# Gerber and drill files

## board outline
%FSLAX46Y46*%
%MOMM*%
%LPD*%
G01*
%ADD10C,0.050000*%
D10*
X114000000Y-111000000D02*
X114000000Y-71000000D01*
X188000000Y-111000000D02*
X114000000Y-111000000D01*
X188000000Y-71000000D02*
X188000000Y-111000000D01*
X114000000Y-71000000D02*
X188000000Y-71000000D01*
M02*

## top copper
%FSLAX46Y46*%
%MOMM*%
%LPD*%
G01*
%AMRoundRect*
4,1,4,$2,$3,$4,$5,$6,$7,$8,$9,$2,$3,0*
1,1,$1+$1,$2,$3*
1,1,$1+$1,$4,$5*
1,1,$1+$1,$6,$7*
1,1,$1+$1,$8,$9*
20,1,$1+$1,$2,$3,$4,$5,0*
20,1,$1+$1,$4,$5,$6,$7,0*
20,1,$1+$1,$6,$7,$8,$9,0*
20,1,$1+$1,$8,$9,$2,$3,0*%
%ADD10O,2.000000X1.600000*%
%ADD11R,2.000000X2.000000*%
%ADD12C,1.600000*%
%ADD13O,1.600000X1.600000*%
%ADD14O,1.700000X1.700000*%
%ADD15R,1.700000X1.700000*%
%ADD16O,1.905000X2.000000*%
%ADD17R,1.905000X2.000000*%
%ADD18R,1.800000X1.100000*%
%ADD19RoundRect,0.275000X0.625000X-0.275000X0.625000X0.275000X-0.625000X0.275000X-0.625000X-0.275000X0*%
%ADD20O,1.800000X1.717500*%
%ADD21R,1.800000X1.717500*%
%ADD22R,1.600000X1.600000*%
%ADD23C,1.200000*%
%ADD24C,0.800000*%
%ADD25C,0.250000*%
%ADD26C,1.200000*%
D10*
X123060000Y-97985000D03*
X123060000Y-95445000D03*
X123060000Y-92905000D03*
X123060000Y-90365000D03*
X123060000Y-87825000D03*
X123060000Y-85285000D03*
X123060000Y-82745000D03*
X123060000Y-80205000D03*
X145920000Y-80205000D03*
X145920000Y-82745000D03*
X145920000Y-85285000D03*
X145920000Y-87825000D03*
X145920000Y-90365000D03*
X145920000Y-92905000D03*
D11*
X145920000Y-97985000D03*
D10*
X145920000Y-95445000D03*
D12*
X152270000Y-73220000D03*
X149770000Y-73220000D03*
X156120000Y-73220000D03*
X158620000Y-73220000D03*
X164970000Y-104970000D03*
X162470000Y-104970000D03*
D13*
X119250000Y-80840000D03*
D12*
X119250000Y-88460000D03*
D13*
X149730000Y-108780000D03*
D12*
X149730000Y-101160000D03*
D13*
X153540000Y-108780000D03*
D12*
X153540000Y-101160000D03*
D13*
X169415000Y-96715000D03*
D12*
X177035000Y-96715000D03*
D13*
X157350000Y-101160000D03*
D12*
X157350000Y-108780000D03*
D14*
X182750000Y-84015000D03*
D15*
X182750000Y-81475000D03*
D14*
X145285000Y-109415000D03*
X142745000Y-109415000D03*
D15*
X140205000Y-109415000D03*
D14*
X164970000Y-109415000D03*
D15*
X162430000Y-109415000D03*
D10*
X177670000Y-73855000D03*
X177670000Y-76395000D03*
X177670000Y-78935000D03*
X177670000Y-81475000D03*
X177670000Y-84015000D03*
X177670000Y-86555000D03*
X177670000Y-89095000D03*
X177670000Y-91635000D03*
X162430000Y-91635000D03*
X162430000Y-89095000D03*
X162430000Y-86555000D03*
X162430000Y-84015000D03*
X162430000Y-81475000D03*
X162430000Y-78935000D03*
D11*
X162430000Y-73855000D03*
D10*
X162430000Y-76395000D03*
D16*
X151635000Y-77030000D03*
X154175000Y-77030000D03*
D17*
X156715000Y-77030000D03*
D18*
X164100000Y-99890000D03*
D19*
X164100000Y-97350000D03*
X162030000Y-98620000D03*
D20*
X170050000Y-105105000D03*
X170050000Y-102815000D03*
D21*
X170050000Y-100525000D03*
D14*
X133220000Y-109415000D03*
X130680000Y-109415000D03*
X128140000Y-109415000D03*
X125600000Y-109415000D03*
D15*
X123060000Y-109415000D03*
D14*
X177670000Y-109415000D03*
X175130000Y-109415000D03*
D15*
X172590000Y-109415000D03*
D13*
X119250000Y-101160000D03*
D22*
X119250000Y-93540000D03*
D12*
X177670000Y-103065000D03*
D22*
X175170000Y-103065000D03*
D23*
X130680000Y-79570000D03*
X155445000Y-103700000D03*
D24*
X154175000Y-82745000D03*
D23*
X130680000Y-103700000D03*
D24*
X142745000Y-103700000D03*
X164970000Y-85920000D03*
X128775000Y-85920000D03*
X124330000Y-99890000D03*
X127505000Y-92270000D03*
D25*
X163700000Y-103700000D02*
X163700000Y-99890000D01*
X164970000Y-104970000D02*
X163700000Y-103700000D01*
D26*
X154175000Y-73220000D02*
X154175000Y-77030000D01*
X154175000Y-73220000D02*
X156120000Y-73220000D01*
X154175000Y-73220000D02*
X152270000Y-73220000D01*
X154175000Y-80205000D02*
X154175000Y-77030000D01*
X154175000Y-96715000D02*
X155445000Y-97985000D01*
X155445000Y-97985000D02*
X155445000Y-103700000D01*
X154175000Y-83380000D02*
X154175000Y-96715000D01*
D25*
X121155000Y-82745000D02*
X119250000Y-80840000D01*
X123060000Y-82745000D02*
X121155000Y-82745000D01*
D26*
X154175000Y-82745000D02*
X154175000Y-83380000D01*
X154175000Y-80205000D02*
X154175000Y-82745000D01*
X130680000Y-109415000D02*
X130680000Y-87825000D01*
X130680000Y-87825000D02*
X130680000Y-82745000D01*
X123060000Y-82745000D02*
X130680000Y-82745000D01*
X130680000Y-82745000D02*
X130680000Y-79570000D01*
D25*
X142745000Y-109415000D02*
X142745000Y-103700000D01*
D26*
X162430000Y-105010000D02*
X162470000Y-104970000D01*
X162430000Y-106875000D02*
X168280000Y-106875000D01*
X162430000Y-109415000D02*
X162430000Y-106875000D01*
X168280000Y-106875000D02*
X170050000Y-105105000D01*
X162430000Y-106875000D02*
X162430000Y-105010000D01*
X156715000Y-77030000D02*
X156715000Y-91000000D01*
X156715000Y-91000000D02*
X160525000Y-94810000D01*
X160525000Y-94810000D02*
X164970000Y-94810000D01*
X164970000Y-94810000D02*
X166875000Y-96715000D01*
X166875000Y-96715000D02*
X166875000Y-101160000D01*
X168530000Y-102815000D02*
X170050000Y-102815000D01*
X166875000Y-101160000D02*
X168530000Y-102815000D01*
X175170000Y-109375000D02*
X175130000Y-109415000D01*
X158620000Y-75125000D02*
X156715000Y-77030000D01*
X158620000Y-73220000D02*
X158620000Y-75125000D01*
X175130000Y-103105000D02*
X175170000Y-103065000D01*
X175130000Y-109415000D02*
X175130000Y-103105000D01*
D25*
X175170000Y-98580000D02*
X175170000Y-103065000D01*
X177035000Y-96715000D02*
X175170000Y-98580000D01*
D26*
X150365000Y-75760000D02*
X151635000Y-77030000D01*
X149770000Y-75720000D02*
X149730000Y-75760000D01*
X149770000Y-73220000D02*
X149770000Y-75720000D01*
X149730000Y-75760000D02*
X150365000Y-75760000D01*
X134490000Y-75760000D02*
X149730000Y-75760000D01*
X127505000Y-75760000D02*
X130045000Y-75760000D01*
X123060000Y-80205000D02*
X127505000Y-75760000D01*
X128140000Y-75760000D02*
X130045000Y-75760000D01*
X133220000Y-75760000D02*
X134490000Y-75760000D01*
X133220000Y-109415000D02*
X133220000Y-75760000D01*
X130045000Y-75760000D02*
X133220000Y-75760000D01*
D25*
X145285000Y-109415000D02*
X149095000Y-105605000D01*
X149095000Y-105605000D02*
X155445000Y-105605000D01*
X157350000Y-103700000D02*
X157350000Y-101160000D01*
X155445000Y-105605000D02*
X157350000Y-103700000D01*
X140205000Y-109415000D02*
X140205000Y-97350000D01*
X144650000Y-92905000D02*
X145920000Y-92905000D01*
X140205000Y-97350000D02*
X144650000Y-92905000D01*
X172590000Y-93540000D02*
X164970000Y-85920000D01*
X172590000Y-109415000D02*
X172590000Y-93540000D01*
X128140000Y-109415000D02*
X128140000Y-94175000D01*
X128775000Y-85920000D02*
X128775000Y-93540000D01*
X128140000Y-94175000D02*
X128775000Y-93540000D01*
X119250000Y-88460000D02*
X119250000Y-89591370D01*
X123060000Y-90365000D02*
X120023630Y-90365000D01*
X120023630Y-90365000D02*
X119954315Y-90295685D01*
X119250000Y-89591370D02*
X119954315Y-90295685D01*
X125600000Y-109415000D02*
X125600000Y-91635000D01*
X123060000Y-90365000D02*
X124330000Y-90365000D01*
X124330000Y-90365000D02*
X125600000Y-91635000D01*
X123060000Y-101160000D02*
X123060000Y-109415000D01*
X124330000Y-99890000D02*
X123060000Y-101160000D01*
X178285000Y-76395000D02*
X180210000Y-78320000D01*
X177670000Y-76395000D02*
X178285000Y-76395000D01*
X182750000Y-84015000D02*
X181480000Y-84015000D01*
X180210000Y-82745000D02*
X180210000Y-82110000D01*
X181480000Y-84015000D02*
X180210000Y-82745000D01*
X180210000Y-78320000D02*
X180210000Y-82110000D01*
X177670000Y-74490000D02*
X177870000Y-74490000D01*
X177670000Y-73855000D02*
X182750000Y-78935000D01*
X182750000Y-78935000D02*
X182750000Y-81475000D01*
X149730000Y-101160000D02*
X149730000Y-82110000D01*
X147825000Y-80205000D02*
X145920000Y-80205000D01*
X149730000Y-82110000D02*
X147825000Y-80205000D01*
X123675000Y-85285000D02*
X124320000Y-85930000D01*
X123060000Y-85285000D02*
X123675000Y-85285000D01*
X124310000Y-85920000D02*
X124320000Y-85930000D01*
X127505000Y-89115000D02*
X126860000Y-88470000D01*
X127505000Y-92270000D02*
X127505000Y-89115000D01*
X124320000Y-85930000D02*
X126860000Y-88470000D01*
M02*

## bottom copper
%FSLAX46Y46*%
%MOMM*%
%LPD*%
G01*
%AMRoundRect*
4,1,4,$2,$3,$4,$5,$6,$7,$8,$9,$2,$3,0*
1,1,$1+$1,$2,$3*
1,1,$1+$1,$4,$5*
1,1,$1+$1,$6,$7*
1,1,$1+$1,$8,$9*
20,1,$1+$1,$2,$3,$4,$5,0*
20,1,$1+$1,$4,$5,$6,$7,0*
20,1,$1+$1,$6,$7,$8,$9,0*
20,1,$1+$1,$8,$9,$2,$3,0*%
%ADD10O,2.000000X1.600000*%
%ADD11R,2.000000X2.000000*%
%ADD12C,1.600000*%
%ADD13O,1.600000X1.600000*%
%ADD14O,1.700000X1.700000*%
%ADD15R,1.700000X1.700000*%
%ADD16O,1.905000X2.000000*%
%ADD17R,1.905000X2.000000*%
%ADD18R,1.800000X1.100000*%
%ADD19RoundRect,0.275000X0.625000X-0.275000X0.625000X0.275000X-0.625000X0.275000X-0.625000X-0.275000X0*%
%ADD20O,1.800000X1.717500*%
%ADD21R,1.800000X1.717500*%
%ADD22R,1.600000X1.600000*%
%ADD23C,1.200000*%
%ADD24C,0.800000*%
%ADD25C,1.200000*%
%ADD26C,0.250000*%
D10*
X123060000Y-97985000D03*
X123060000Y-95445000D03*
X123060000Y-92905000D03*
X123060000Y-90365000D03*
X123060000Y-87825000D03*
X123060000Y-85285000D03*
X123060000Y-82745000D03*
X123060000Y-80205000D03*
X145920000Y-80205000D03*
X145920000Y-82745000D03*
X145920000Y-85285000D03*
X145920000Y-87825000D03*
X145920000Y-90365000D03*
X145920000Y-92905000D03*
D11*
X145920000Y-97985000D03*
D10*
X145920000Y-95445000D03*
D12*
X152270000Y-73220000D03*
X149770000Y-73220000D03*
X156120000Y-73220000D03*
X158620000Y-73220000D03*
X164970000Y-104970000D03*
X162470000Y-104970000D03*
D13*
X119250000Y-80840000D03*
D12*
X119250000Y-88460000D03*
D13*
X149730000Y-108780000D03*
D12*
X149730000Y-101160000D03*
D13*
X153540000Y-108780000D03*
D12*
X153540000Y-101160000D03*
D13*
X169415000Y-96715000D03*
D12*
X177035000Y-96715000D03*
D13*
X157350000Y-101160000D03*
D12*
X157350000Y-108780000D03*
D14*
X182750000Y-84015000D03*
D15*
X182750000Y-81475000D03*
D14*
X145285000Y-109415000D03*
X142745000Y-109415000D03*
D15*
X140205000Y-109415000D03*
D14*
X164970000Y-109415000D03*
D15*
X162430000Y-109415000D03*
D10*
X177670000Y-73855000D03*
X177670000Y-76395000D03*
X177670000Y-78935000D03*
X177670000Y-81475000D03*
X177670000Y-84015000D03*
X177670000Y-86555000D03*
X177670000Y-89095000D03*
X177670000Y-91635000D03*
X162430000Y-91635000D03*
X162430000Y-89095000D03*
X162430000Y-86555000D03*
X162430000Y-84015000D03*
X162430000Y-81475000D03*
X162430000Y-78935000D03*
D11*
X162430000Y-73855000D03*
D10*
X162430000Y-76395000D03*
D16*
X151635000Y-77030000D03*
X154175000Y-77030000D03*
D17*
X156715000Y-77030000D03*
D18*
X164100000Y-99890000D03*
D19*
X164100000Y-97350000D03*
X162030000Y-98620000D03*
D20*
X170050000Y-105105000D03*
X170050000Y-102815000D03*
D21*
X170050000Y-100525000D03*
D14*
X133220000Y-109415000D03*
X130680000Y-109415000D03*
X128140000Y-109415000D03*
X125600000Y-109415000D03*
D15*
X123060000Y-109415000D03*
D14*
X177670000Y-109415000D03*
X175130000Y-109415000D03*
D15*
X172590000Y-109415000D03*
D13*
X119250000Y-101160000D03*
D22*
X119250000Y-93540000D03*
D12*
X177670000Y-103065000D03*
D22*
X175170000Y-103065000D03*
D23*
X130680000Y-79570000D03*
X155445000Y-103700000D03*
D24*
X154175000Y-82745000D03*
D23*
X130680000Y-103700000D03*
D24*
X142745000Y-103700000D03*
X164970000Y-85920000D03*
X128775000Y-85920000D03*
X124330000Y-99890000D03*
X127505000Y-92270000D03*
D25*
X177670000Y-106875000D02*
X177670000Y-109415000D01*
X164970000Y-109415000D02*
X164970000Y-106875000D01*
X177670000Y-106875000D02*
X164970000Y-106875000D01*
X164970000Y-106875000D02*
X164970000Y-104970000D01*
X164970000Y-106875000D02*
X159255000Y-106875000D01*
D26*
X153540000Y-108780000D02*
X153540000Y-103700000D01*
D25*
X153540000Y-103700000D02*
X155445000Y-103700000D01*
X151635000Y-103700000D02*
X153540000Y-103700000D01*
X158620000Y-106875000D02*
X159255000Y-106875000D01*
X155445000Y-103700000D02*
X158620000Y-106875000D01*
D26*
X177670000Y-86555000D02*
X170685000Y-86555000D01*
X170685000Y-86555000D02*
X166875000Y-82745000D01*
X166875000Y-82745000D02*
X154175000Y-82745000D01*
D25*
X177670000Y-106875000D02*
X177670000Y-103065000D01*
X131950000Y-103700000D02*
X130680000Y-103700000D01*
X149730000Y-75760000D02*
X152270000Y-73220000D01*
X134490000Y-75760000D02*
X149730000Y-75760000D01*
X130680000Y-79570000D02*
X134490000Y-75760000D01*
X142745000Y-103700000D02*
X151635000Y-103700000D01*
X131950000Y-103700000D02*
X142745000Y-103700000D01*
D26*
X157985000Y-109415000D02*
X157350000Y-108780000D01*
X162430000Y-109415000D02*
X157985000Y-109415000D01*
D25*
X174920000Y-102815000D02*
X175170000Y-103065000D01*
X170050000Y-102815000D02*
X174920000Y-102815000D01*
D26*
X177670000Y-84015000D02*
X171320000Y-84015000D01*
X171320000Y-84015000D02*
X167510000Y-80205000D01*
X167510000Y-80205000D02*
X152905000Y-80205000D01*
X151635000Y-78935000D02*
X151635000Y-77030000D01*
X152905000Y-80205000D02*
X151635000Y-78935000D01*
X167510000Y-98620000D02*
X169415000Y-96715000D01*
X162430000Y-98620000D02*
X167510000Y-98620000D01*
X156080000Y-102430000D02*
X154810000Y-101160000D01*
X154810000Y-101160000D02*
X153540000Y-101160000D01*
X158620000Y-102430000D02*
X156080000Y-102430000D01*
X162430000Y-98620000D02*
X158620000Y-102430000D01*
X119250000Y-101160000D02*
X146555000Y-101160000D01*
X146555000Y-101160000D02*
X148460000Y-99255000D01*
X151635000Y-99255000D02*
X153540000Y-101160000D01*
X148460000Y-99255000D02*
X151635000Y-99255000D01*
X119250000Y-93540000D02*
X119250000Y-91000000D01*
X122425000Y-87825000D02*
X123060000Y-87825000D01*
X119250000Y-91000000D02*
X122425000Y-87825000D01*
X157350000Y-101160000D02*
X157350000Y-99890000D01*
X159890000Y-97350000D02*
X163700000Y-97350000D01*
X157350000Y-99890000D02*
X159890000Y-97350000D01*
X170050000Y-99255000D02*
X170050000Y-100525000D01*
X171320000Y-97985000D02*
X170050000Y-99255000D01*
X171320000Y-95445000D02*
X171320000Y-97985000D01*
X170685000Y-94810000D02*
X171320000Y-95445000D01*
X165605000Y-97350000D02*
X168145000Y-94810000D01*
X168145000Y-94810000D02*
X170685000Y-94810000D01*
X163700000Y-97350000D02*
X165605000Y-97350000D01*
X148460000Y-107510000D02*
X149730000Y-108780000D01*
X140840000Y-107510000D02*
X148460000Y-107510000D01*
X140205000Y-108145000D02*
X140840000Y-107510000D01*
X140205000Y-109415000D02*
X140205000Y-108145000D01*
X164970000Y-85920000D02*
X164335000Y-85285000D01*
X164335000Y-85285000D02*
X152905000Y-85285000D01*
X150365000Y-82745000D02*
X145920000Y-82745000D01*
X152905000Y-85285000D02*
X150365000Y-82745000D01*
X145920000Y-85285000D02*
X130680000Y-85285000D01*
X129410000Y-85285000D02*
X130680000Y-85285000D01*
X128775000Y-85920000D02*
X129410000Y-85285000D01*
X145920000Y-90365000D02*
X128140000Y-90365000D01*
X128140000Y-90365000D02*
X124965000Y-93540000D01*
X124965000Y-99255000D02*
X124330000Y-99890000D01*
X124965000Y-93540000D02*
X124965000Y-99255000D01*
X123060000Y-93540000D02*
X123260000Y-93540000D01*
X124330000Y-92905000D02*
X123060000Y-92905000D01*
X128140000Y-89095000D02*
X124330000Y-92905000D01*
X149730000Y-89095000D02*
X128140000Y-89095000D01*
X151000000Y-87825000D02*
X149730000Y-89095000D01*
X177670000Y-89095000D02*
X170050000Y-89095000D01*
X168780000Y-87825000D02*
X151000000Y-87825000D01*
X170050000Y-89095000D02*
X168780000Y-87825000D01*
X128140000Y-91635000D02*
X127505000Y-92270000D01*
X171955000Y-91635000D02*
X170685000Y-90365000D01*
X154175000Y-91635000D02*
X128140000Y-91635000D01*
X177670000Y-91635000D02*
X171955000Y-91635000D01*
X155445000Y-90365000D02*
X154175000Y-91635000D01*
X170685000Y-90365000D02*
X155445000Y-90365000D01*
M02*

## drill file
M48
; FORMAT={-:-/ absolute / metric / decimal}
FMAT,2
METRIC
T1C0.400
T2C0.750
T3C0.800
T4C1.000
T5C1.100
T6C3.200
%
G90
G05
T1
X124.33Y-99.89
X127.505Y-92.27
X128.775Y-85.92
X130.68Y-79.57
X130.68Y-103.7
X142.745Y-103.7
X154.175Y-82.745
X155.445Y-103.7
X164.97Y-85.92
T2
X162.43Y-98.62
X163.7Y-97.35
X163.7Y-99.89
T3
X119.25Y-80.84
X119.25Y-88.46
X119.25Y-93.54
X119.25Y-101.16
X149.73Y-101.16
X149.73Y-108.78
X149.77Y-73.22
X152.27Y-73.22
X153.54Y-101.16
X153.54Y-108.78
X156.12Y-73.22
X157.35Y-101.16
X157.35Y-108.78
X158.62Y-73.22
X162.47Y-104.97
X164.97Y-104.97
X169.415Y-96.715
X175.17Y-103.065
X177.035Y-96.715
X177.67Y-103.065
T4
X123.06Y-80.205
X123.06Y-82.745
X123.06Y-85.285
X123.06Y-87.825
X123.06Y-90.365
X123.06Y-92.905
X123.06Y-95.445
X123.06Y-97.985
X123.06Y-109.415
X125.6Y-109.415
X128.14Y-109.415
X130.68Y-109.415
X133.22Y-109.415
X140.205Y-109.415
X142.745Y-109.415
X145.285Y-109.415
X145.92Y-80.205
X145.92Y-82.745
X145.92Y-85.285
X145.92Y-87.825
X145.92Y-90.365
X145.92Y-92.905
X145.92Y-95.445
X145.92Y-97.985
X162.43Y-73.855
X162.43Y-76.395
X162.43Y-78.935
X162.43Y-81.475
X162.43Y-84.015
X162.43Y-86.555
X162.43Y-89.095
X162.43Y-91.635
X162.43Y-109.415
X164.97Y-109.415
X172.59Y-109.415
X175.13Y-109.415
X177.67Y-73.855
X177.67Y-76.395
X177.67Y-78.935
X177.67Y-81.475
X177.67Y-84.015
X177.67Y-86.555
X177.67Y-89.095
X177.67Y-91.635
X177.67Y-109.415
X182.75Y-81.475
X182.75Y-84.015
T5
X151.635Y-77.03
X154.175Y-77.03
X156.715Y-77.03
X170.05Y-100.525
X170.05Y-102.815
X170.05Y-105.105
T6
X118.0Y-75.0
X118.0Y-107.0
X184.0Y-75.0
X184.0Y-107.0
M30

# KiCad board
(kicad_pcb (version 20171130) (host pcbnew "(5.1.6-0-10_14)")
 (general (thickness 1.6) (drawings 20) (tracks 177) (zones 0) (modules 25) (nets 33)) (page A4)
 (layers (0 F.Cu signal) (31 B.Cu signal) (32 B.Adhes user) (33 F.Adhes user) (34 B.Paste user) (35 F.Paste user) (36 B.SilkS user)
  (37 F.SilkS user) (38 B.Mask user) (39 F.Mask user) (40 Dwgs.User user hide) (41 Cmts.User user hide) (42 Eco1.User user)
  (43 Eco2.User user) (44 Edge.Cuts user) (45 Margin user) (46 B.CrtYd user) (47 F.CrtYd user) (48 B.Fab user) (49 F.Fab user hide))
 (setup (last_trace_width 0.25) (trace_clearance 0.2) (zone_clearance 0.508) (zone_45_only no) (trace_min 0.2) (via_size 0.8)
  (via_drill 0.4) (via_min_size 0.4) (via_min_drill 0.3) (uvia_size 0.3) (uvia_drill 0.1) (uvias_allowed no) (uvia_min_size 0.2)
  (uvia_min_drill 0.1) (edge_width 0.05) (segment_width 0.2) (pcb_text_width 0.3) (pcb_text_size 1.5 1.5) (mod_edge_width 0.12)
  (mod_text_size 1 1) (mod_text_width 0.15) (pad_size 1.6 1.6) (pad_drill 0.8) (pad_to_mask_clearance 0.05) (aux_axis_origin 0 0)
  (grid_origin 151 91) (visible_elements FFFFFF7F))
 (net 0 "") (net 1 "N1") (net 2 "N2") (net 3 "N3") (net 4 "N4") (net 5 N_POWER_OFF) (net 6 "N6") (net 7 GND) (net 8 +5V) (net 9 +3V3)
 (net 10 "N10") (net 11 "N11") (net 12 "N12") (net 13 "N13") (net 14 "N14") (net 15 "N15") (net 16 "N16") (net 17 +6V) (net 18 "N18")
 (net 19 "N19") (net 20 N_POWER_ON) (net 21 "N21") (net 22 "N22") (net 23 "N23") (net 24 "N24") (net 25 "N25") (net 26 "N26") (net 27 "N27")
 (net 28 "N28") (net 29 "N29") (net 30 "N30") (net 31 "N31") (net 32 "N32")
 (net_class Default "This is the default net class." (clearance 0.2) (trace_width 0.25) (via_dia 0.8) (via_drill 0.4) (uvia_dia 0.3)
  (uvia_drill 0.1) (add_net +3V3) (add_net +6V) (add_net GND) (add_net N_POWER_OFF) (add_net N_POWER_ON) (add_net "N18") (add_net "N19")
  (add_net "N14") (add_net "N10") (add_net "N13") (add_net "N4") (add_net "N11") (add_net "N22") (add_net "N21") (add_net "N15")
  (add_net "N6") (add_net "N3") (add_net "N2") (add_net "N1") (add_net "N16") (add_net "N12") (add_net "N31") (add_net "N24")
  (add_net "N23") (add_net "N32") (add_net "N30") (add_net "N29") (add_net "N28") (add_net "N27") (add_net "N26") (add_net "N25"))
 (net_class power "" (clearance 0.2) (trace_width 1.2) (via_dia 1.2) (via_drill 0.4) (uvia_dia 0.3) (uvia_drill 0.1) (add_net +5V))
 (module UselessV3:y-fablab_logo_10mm (layer F.Cu) (at 154.175 88.46)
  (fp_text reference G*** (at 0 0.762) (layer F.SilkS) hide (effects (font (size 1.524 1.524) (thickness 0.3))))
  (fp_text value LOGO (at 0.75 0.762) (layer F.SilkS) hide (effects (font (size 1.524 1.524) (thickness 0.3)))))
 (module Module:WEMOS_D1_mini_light (layer F.Cu) (at 145.92 97.985 180)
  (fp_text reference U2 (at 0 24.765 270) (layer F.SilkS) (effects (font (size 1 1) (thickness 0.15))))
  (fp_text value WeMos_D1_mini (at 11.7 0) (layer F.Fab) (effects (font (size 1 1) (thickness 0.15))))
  (pad 16 thru_hole oval (at 22.86 0 180) (size 2 1.6) (drill 1) (layers *.Cu *.Mask) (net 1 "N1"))
  (pad 15 thru_hole oval (at 22.86 2.54 180) (size 2 1.6) (drill 1) (layers *.Cu *.Mask) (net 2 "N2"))
  (pad 14 thru_hole oval (at 22.86 5.08 180) (size 2 1.6) (drill 1) (layers *.Cu *.Mask) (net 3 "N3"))
  (pad 13 thru_hole oval (at 22.86 7.62 180) (size 2 1.6) (drill 1) (layers *.Cu *.Mask) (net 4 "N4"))
  (pad 12 thru_hole oval (at 22.86 10.16 180) (size 2 1.6) (drill 1) (layers *.Cu *.Mask) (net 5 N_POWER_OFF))
  (pad 11 thru_hole oval (at 22.86 12.7 180) (size 2 1.6) (drill 1) (layers *.Cu *.Mask) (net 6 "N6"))
  (pad 10 thru_hole oval (at 22.86 15.24 180) (size 2 1.6) (drill 1) (layers *.Cu *.Mask) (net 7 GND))
  (pad 9 thru_hole oval (at 22.86 17.78 180) (size 2 1.6) (drill 1) (layers *.Cu *.Mask) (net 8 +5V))
  (pad 8 thru_hole oval (at 0 17.78 180) (size 2 1.6) (drill 1) (layers *.Cu *.Mask) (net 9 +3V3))
  (pad 7 thru_hole oval (at 0 15.24 180) (size 2 1.6) (drill 1) (layers *.Cu *.Mask) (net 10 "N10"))
  (pad 6 thru_hole oval (at 0 12.7 180) (size 2 1.6) (drill 1) (layers *.Cu *.Mask) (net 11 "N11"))
  (pad 5 thru_hole oval (at 0 10.16 180) (size 2 1.6) (drill 1) (layers *.Cu *.Mask) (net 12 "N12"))
  (pad 4 thru_hole oval (at 0 7.62 180) (size 2 1.6) (drill 1) (layers *.Cu *.Mask) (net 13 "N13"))
  (pad 3 thru_hole oval (at 0 5.08 180) (size 2 1.6) (drill 1) (layers *.Cu *.Mask) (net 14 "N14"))
  (pad 1 thru_hole rect (at 0 0 180) (size 2 2) (drill 1) (layers *.Cu *.Mask) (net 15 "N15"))
  (pad 2 thru_hole oval (at 0 2.54 180) (size 2 1.6) (drill 1) (layers *.Cu *.Mask) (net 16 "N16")))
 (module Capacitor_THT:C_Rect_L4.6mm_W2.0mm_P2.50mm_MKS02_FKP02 (layer F.Cu) (at 149.77 73.22)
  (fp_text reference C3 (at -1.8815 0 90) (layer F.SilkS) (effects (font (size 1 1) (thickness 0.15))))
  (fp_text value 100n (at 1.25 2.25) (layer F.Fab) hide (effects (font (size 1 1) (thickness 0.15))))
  (pad 2 thru_hole circle (at 2.5 0) (size 1.6 1.6) (drill 0.8) (layers *.Cu *.Mask) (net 7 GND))
  (pad 1 thru_hole circle (at 0 0) (size 1.6 1.6) (drill 0.8) (layers *.Cu *.Mask) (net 8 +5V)))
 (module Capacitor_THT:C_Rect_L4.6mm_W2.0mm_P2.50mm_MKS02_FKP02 (layer F.Cu) (at 158.62 73.22 180)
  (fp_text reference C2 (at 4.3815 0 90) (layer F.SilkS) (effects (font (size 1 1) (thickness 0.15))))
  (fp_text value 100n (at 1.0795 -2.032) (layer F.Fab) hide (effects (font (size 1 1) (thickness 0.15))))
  (pad 2 thru_hole circle (at 2.5 0 180) (size 1.6 1.6) (drill 0.8) (layers *.Cu *.Mask) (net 7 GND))
  (pad 1 thru_hole circle (at 0 0 180) (size 1.6 1.6) (drill 0.8) (layers *.Cu *.Mask) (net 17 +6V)))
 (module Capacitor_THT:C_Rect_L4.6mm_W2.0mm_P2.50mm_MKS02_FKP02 (layer F.Cu) (at 162.47 104.97)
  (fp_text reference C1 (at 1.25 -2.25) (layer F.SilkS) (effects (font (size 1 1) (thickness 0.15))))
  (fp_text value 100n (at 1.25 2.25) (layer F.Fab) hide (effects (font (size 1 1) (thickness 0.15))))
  (pad 2 thru_hole circle (at 2.5 0) (size 1.6 1.6) (drill 0.8) (layers *.Cu *.Mask) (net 7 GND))
  (pad 1 thru_hole circle (at 0 0) (size 1.6 1.6) (drill 0.8) (layers *.Cu *.Mask) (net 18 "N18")))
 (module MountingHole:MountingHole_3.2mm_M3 (layer F.Cu) (at 184 75)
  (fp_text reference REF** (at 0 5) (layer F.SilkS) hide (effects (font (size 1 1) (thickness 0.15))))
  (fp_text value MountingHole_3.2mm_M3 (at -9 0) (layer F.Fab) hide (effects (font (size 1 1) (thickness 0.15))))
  (pad 1 np_thru_hole circle (at 0 0) (size 3.2 3.2) (drill 3.2) (layers *.Cu *.Mask)))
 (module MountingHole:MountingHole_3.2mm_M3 (layer F.Cu) (at 184 107)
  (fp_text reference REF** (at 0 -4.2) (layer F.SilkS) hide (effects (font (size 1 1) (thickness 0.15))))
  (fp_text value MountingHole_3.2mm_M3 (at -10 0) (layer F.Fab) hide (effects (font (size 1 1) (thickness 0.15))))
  (pad 1 np_thru_hole circle (at 0 0) (size 3.2 3.2) (drill 3.2) (layers *.Cu *.Mask)))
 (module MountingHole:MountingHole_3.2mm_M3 (layer F.Cu) (at 118 107)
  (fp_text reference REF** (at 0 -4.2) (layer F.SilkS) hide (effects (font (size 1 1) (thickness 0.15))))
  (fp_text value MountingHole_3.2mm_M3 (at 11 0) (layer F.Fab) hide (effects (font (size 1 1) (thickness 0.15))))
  (pad 1 np_thru_hole circle (at 0 0) (size 3.2 3.2) (drill 3.2) (layers *.Cu *.Mask)))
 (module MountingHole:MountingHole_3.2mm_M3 (layer F.Cu) (at 118 75)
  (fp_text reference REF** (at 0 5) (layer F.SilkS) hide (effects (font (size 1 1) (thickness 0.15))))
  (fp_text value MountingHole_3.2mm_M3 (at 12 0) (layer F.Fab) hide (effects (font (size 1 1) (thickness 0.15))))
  (pad 1 np_thru_hole circle (at 0 0) (size 3.2 3.2) (drill 3.2) (layers *.Cu *.Mask)))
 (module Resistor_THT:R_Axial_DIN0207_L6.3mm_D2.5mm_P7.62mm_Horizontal (layer F.Cu) (at 119.25 88.46 90)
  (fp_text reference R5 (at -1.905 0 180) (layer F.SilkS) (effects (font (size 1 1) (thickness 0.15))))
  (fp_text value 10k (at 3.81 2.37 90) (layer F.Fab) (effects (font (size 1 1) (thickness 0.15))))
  (pad 2 thru_hole oval (at 7.62 0 90) (size 1.6 1.6) (drill 0.8) (layers *.Cu *.Mask) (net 7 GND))
  (pad 1 thru_hole circle (at 0 0 90) (size 1.6 1.6) (drill 0.8) (layers *.Cu *.Mask) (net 4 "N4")))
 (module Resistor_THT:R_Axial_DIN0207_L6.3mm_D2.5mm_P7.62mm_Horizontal (layer F.Cu) (at 149.73 101.16 270)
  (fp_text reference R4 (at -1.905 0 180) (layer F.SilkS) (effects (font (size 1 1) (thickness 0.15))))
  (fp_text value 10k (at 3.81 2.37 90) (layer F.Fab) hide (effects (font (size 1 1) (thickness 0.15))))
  (pad 2 thru_hole oval (at 7.62 0 270) (size 1.6 1.6) (drill 0.8) (layers *.Cu *.Mask) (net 14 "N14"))
  (pad 1 thru_hole circle (at 0 0 270) (size 1.6 1.6) (drill 0.8) (layers *.Cu *.Mask) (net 9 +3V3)))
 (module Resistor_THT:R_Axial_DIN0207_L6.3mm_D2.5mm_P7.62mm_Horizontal (layer F.Cu) (at 153.54 101.16 270)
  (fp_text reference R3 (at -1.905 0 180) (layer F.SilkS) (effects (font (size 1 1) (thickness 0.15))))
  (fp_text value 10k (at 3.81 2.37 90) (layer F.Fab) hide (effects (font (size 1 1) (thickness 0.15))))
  (pad 2 thru_hole oval (at 7.62 0 270) (size 1.6 1.6) (drill 0.8) (layers *.Cu *.Mask) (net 7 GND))
  (pad 1 thru_hole circle (at 0 0 270) (size 1.6 1.6) (drill 0.8) (layers *.Cu *.Mask) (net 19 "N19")))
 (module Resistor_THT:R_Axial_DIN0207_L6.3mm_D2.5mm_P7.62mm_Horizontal (layer F.Cu) (at 177.035 96.715 180)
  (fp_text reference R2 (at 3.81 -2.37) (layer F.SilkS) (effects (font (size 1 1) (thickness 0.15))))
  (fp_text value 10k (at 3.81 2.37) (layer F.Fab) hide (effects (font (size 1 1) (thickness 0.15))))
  (pad 2 thru_hole oval (at 7.62 0 180) (size 1.6 1.6) (drill 0.8) (layers *.Cu *.Mask) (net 19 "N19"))
  (pad 1 thru_hole circle (at 0 0 180) (size 1.6 1.6) (drill 0.8) (layers *.Cu *.Mask) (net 17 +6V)))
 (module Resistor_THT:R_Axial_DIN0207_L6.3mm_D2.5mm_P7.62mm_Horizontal (layer F.Cu) (at 157.35 108.78 90)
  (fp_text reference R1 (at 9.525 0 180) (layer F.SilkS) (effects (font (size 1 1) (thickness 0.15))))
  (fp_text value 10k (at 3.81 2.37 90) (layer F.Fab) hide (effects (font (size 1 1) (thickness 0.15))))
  (pad 2 thru_hole oval (at 7.62 0 90) (size 1.6 1.6) (drill 0.8) (layers *.Cu *.Mask) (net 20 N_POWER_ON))
  (pad 1 thru_hole circle (at 0 0 90) (size 1.6 1.6) (drill 0.8) (layers *.Cu *.Mask) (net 18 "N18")))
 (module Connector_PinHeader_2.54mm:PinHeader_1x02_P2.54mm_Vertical (layer F.Cu) (at 182.75 81.475)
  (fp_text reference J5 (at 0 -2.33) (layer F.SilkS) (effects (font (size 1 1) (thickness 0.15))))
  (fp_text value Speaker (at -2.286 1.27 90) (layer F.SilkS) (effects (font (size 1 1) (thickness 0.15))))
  (pad 2 thru_hole oval (at 0 2.54) (size 1.7 1.7) (drill 1) (layers *.Cu *.Mask) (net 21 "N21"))
  (pad 1 thru_hole rect (at 0 0) (size 1.7 1.7) (drill 1) (layers *.Cu *.Mask) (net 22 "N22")))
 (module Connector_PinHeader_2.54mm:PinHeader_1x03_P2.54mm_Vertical (layer F.Cu) (at 140.205 109.415 90)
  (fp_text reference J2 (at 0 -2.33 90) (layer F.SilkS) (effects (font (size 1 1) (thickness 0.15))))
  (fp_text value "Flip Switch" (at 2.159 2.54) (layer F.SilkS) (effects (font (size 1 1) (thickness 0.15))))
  (pad 3 thru_hole oval (at 0 5.08 90) (size 1.7 1.7) (drill 1) (layers *.Cu *.Mask) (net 20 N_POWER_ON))
  (pad 2 thru_hole oval (at 0 2.54 90) (size 1.7 1.7) (drill 1) (layers *.Cu *.Mask) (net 7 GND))
  (pad 1 thru_hole rect (at 0 0 90) (size 1.7 1.7) (drill 1) (layers *.Cu *.Mask) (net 14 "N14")))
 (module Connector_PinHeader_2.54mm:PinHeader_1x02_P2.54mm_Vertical (layer F.Cu) (at 162.43 109.415 90)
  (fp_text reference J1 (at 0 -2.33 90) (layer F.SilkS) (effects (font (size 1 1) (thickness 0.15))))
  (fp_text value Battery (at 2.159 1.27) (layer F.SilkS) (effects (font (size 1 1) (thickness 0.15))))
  (pad 2 thru_hole oval (at 0 2.54 90) (size 1.7 1.7) (drill 1) (layers *.Cu *.Mask) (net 7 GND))
  (pad 1 thru_hole rect (at 0 0 90) (size 1.7 1.7) (drill 1) (layers *.Cu *.Mask) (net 18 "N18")))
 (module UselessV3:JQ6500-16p (layer F.Cu) (at 162.43 73.855)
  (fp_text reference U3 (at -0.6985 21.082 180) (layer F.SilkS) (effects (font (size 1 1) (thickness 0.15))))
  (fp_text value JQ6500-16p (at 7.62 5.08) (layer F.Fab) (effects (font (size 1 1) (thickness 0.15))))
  (pad 16 thru_hole oval (at 15.24 0) (size 2 1.6) (drill 1) (layers *.Cu *.Mask) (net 22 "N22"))
  (pad 15 thru_hole oval (at 15.24 2.54) (size 2 1.6) (drill 1) (layers *.Cu *.Mask) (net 21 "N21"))
  (pad 14 thru_hole oval (at 15.24 5.08) (size 2 1.6) (drill 1) (layers *.Cu *.Mask) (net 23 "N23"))
  (pad 13 thru_hole oval (at 15.24 7.62) (size 2 1.6) (drill 1) (layers *.Cu *.Mask) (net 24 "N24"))
  (pad 12 thru_hole oval (at 15.24 10.16) (size 2 1.6) (drill 1) (layers *.Cu *.Mask) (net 8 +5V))
  (pad 11 thru_hole oval (at 15.24 12.7) (size 2 1.6) (drill 1) (layers *.Cu *.Mask) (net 7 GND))
  (pad 10 thru_hole oval (at 15.24 15.24) (size 2 1.6) (drill 1) (layers *.Cu *.Mask) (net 3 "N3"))
  (pad 9 thru_hole oval (at 15.24 17.78) (size 2 1.6) (drill 1) (layers *.Cu *.Mask) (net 6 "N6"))
  (pad 8 thru_hole oval (at 0 17.78) (size 2 1.6) (drill 1) (layers *.Cu *.Mask) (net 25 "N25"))
  (pad 7 thru_hole oval (at 0 15.24) (size 2 1.6) (drill 1) (layers *.Cu *.Mask) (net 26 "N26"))
  (pad 6 thru_hole oval (at 0 12.7) (size 2 1.6) (drill 1) (layers *.Cu *.Mask) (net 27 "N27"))
  (pad 5 thru_hole oval (at 0 10.16) (size 2 1.6) (drill 1) (layers *.Cu *.Mask) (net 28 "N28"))
  (pad 4 thru_hole oval (at 0 7.62) (size 2 1.6) (drill 1) (layers *.Cu *.Mask) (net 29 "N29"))
  (pad 3 thru_hole oval (at 0 5.08) (size 2 1.6) (drill 1) (layers *.Cu *.Mask) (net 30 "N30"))
  (pad 1 thru_hole rect (at 0 0) (size 2 2) (drill 1) (layers *.Cu *.Mask) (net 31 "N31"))
  (pad 2 thru_hole oval (at 0 2.54) (size 2 1.6) (drill 1) (layers *.Cu *.Mask) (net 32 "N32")))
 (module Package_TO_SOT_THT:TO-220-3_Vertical (layer F.Cu) (at 156.715 77.03 180)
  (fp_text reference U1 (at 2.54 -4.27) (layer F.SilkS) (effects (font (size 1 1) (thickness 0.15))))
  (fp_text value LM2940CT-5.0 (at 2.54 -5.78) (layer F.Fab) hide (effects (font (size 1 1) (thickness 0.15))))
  (pad 3 thru_hole oval (at 5.08 0 180) (size 1.905 2) (drill 1.1) (layers *.Cu *.Mask) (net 8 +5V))
  (pad 2 thru_hole oval (at 2.54 0 180) (size 1.905 2) (drill 1.1) (layers *.Cu *.Mask) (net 7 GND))
  (pad 1 thru_hole rect (at 0 0 180) (size 1.905 2) (drill 1.1) (layers *.Cu *.Mask) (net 17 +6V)))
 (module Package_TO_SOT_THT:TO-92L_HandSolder (layer F.Cu) (at 163.7 99.89 90)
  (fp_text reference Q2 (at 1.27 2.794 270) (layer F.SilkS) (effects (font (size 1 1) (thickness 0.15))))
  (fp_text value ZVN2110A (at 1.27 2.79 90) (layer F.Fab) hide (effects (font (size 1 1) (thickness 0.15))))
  (pad 1 thru_hole rect (at 0 0 90) (size 1.1 1.8) (drill 0.75 (offset 0 0.4)) (layers *.Cu *.Mask) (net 7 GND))
  (pad 3 thru_hole roundrect (at 2.54 0 90) (size 1.1 1.8) (drill 0.75 (offset 0 0.4)) (layers *.Cu *.Mask) (roundrect_rratio 0.25)
   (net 20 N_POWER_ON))
  (pad 2 thru_hole roundrect (at 1.27 -1.27 90) (size 1.1 1.8) (drill 0.75 (offset 0 -0.4)) (layers *.Cu *.Mask) (roundrect_rratio 0.25)
   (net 19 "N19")))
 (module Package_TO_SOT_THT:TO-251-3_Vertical (layer F.Cu) (at 170.05 100.525 270)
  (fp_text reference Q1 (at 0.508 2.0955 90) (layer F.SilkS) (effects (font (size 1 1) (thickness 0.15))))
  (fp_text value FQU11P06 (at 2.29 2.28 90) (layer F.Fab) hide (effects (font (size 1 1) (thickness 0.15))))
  (pad 3 thru_hole oval (at 4.58 0 270) (size 1.7175 1.8) (drill 1.1) (layers *.Cu *.Mask) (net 18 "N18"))
  (pad 2 thru_hole oval (at 2.29 0 270) (size 1.7175 1.8) (drill 1.1) (layers *.Cu *.Mask) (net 17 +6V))
  (pad 1 thru_hole rect (at 0 0 270) (size 1.7175 1.8) (drill 1.1) (layers *.Cu *.Mask) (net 20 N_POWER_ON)))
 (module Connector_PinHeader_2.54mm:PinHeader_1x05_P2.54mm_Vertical (layer F.Cu) (at 123.06 109.415 90)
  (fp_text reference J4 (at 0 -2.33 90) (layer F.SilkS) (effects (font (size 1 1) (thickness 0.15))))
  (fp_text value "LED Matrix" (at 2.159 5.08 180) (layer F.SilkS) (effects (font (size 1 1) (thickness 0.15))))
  (pad 5 thru_hole oval (at 0 10.16 90) (size 1.7 1.7) (drill 1) (layers *.Cu *.Mask) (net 8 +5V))
  (pad 4 thru_hole oval (at 0 7.62 90) (size 1.7 1.7) (drill 1) (layers *.Cu *.Mask) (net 7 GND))
  (pad 3 thru_hole oval (at 0 5.08 90) (size 1.7 1.7) (drill 1) (layers *.Cu *.Mask) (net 11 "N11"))
  (pad 2 thru_hole oval (at 0 2.54 90) (size 1.7 1.7) (drill 1) (layers *.Cu *.Mask) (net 4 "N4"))
  (pad 1 thru_hole rect (at 0 0 90) (size 1.7 1.7) (drill 1) (layers *.Cu *.Mask) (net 13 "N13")))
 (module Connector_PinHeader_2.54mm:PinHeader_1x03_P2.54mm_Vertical (layer F.Cu) (at 172.59 109.415 90)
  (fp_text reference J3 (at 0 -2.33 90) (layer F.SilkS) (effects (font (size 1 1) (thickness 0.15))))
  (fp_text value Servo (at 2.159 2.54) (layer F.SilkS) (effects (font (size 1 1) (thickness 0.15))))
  (pad 3 thru_hole oval (at 0 5.08 90) (size 1.7 1.7) (drill 1) (layers *.Cu *.Mask) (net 7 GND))
  (pad 2 thru_hole oval (at 0 2.54 90) (size 1.7 1.7) (drill 1) (layers *.Cu *.Mask) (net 17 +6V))
  (pad 1 thru_hole rect (at 0 0 90) (size 1.7 1.7) (drill 1) (layers *.Cu *.Mask) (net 10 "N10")))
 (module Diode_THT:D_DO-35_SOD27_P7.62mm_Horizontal (layer F.Cu) (at 119.25 93.54 270)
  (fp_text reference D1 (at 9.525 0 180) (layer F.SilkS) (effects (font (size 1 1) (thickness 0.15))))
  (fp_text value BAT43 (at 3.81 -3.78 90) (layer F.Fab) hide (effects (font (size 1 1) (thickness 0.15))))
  (pad 2 thru_hole oval (at 7.62 0 270) (size 1.6 1.6) (drill 0.8) (layers *.Cu *.Mask) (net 19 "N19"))
  (pad 1 thru_hole rect (at 0 0 270) (size 1.6 1.6) (drill 0.8) (layers *.Cu *.Mask) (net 5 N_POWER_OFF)))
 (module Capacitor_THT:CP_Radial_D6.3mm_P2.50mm (layer F.Cu) (at 175.17 103.065)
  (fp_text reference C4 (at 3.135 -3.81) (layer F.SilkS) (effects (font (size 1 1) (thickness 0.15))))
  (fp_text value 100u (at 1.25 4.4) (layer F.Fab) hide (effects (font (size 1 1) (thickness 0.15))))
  (pad 2 thru_hole circle (at 2.5 0) (size 1.6 1.6) (drill 0.8) (layers *.Cu *.Mask) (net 7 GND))
  (pad 1 thru_hole rect (at 0 0) (size 1.6 1.6) (drill 0.8) (layers *.Cu *.Mask) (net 17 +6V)))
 (gr_line (start 114 111) (end 114 71) (layer Edge.Cuts) (width 0.05))
 (gr_line (start 188 111) (end 114 111) (layer Edge.Cuts) (width 0.05))
 (gr_line (start 188 71) (end 188 111) (layer Edge.Cuts) (width 0.05))
 (gr_line (start 114 71) (end 188 71) (layer Edge.Cuts) (width 0.05))
 (segment (start 163.7 103.7) (end 163.7 99.89) (width 0.25) (layer F.Cu) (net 7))
 (segment (start 164.97 104.97) (end 163.7 103.7) (width 0.25) (layer F.Cu) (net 7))
 (segment (start 177.67 106.875) (end 177.67 109.415) (width 1.2) (layer B.Cu) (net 7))
 (segment (start 164.97 109.415) (end 164.97 106.875) (width 1.2) (layer B.Cu) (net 7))
 (segment (start 177.67 106.875) (end 164.97 106.875) (width 1.2) (layer B.Cu) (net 7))
 (segment (start 164.97 106.875) (end 164.97 104.97) (width 1.2) (layer B.Cu) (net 7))
 (segment (start 154.175 73.22) (end 154.175 77.03) (width 1.2) (layer F.Cu) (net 7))
 (segment (start 154.175 73.22) (end 156.12 73.22) (width 1.2) (layer F.Cu) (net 7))
 (segment (start 154.175 73.22) (end 152.27 73.22) (width 1.2) (layer F.Cu) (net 7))
 (via (at 130.68 79.57) (size 1.2) (drill 0.4) (layers F.Cu B.Cu) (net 7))
 (segment (start 154.175 80.205) (end 154.175 77.03) (width 1.2) (layer F.Cu) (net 7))
 (segment (start 154.175 96.715) (end 155.445 97.985) (width 1.2) (layer F.Cu) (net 7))
 (via (at 155.445 103.7) (size 1.2) (drill 0.4) (layers F.Cu B.Cu) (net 7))
 (segment (start 155.445 97.985) (end 155.445 103.7) (width 1.2) (layer F.Cu) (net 7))
 (segment (start 154.175 83.38) (end 154.175 96.715) (width 1.2) (layer F.Cu) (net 7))
 (segment (start 164.97 106.875) (end 159.255 106.875) (width 1.2) (layer B.Cu) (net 7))
 (segment (start 153.54 108.78) (end 153.54 103.7) (width 0.25) (layer B.Cu) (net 7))
 (segment (start 153.54 103.7) (end 155.445 103.7) (width 1.2) (layer B.Cu) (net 7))
 (segment (start 151.635 103.7) (end 153.54 103.7) (width 1.2) (layer B.Cu) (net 7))
 (segment (start 158.62 106.875) (end 159.255 106.875) (width 1.2) (layer B.Cu) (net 7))
 (segment (start 155.445 103.7) (end 158.62 106.875) (width 1.2) (layer B.Cu) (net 7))
 (segment (start 121.155 82.745) (end 119.25 80.84) (width 0.25) (layer F.Cu) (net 7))
 (segment (start 123.06 82.745) (end 121.155 82.745) (width 0.25) (layer F.Cu) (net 7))
 (segment (start 177.67 86.555) (end 170.685 86.555) (width 0.25) (layer B.Cu) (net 7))
 (segment (start 170.685 86.555) (end 166.875 82.745) (width 0.25) (layer B.Cu) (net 7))
 (segment (start 154.175 82.745) (end 154.175 83.38) (width 1.2) (layer F.Cu) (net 7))
 (via (at 154.175 82.745) (size 0.8) (drill 0.4) (layers F.Cu B.Cu) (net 7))
 (segment (start 166.875 82.745) (end 154.175 82.745) (width 0.25) (layer B.Cu) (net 7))
 (segment (start 154.175 80.205) (end 154.175 82.745) (width 1.2) (layer F.Cu) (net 7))
 (segment (start 177.67 106.875) (end 177.67 103.065) (width 1.2) (layer B.Cu) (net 7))
 (segment (start 130.68 109.415) (end 130.68 87.825) (width 1.2) (layer F.Cu) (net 7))
 (segment (start 130.68 87.825) (end 130.68 82.745) (width 1.2) (layer F.Cu) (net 7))
 (segment (start 123.06 82.745) (end 130.68 82.745) (width 1.2) (layer F.Cu) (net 7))
 (segment (start 130.68 82.745) (end 130.68 79.57) (width 1.2) (layer F.Cu) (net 7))
 (segment (start 131.95 103.7) (end 130.68 103.7) (width 1.2) (layer B.Cu) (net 7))
 (via (at 130.68 103.7) (size 1.2) (drill 0.4) (layers F.Cu B.Cu) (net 7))
 (segment (start 149.73 75.76) (end 152.27 73.22) (width 1.2) (layer B.Cu) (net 7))
 (segment (start 134.49 75.76) (end 149.73 75.76) (width 1.2) (layer B.Cu) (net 7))
 (segment (start 130.68 79.57) (end 134.49 75.76) (width 1.2) (layer B.Cu) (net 7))
 (via (at 142.745 103.7) (size 0.8) (drill 0.4) (layers F.Cu B.Cu) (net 7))
 (segment (start 142.745 109.415) (end 142.745 103.7) (width 0.25) (layer F.Cu) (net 7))
 (segment (start 142.745 103.7) (end 151.635 103.7) (width 1.2) (layer B.Cu) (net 7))
 (segment (start 131.95 103.7) (end 142.745 103.7) (width 1.2) (layer B.Cu) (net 7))
 (segment (start 162.43 105.01) (end 162.47 104.97) (width 1.2) (layer F.Cu) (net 18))
 (segment (start 162.43 106.875) (end 168.28 106.875) (width 1.2) (layer F.Cu) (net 18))
 (segment (start 162.43 109.415) (end 162.43 106.875) (width 1.2) (layer F.Cu) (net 18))
 (segment (start 168.28 106.875) (end 170.05 105.105) (width 1.2) (layer F.Cu) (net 18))
 (segment (start 162.43 106.875) (end 162.43 105.01) (width 1.2) (layer F.Cu) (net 18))
 (segment (start 157.985 109.415) (end 157.35 108.78) (width 0.25) (layer B.Cu) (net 18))
 (segment (start 162.43 109.415) (end 157.985 109.415) (width 0.25) (layer B.Cu) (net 18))
 (segment (start 156.715 77.03) (end 156.715 91) (width 1.2) (layer F.Cu) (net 17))
 (segment (start 156.715 91) (end 160.525 94.81) (width 1.2) (layer F.Cu) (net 17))
 (segment (start 160.525 94.81) (end 164.97 94.81) (width 1.2) (layer F.Cu) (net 17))
 (segment (start 164.97 94.81) (end 166.875 96.715) (width 1.2) (layer F.Cu) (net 17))
 (segment (start 166.875 96.715) (end 166.875 101.16) (width 1.2) (layer F.Cu) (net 17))
 (segment (start 168.53 102.815) (end 170.05 102.815) (width 1.2) (layer F.Cu) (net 17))
 (segment (start 166.875 101.16) (end 168.53 102.815) (width 1.2) (layer F.Cu) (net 17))
 (segment (start 175.17 109.375) (end 175.13 109.415) (width 1.2) (layer F.Cu) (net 17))
 (segment (start 158.62 75.125) (end 156.715 77.03) (width 1.2) (layer F.Cu) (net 17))
 (segment (start 158.62 73.22) (end 158.62 75.125) (width 1.2) (layer F.Cu) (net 17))
 (segment (start 175.13 103.105) (end 175.17 103.065) (width 1.2) (layer F.Cu) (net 17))
 (segment (start 175.13 109.415) (end 175.13 103.105) (width 1.2) (layer F.Cu) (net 17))
 (segment (start 174.92 102.815) (end 175.17 103.065) (width 1.2) (layer B.Cu) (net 17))
 (segment (start 170.05 102.815) (end 174.92 102.815) (width 1.2) (layer B.Cu) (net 17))
 (segment (start 175.17 98.58) (end 175.17 103.065) (width 0.25) (layer F.Cu) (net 17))
 (segment (start 177.035 96.715) (end 175.17 98.58) (width 0.25) (layer F.Cu) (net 17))
 (segment (start 150.365 75.76) (end 151.635 77.03) (width 1.2) (layer F.Cu) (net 8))
 (segment (start 149.77 75.72) (end 149.73 75.76) (width 1.2) (layer F.Cu) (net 8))
 (segment (start 149.77 73.22) (end 149.77 75.72) (width 1.2) (layer F.Cu) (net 8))
 (segment (start 149.73 75.76) (end 150.365 75.76) (width 1.2) (layer F.Cu) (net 8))
 (segment (start 134.49 75.76) (end 149.73 75.76) (width 1.2) (layer F.Cu) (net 8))
 (segment (start 127.505 75.76) (end 130.045 75.76) (width 1.2) (layer F.Cu) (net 8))
 (segment (start 123.06 80.205) (end 127.505 75.76) (width 1.2) (layer F.Cu) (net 8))
 (segment (start 128.14 75.76) (end 130.045 75.76) (width 1.2) (layer F.Cu) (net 8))
 (segment (start 177.67 84.015) (end 171.32 84.015) (width 0.25) (layer B.Cu) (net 8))
 (segment (start 171.32 84.015) (end 167.51 80.205) (width 0.25) (layer B.Cu) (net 8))
 (segment (start 167.51 80.205) (end 152.905 80.205) (width 0.25) (layer B.Cu) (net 8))
 (segment (start 151.635 78.935) (end 151.635 77.03) (width 0.25) (layer B.Cu) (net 8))
 (segment (start 152.905 80.205) (end 151.635 78.935) (width 0.25) (layer B.Cu) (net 8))
 (segment (start 133.22 75.76) (end 134.49 75.76) (width 1.2) (layer F.Cu) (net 8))
 (segment (start 133.22 109.415) (end 133.22 75.76) (width 1.2) (layer F.Cu) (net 8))
 (segment (start 130.045 75.76) (end 133.22 75.76) (width 1.2) (layer F.Cu) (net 8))
 (segment (start 167.51 98.62) (end 169.415 96.715) (width 0.25) (layer B.Cu) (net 19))
 (segment (start 162.43 98.62) (end 167.51 98.62) (width 0.25) (layer B.Cu) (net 19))
 (segment (start 156.08 102.43) (end 154.81 101.16) (width 0.25) (layer B.Cu) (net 19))
 (segment (start 154.81 101.16) (end 153.54 101.16) (width 0.25) (layer B.Cu) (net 19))
 (segment (start 158.62 102.43) (end 156.08 102.43) (width 0.25) (layer B.Cu) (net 19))
 (segment (start 162.43 98.62) (end 158.62 102.43) (width 0.25) (layer B.Cu) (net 19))
 (segment (start 119.25 101.16) (end 146.555 101.16) (width 0.25) (layer B.Cu) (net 19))
 (segment (start 146.555 101.16) (end 148.46 99.255) (width 0.25) (layer B.Cu) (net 19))
 (segment (start 151.635 99.255) (end 153.54 101.16) (width 0.25) (layer B.Cu) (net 19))
 (segment (start 148.46 99.255) (end 151.635 99.255) (width 0.25) (layer B.Cu) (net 19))
 (segment (start 119.25 93.54) (end 119.25 91) (width 0.25) (layer B.Cu) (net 5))
 (segment (start 122.425 87.825) (end 123.06 87.825) (width 0.25) (layer B.Cu) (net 5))
 (segment (start 119.25 91) (end 122.425 87.825) (width 0.25) (layer B.Cu) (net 5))
 (segment (start 157.35 101.16) (end 157.35 99.89) (width 0.25) (layer B.Cu) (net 20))
 (segment (start 159.89 97.35) (end 163.7 97.35) (width 0.25) (layer B.Cu) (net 20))
 (segment (start 157.35 99.89) (end 159.89 97.35) (width 0.25) (layer B.Cu) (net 20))
 (segment (start 170.05 99.255) (end 170.05 100.525) (width 0.25) (layer B.Cu) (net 20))
 (segment (start 171.32 97.985) (end 170.05 99.255) (width 0.25) (layer B.Cu) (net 20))
 (segment (start 171.32 95.445) (end 171.32 97.985) (width 0.25) (layer B.Cu) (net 20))
 (segment (start 170.685 94.81) (end 171.32 95.445) (width 0.25) (layer B.Cu) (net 20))
 (segment (start 165.605 97.35) (end 168.145 94.81) (width 0.25) (layer B.Cu) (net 20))
 (segment (start 168.145 94.81) (end 170.685 94.81) (width 0.25) (layer B.Cu) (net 20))
 (segment (start 163.7 97.35) (end 165.605 97.35) (width 0.25) (layer B.Cu) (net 20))
 (segment (start 145.285 109.415) (end 149.095 105.605) (width 0.25) (layer F.Cu) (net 20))
 (segment (start 149.095 105.605) (end 155.445 105.605) (width 0.25) (layer F.Cu) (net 20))
 (segment (start 157.35 103.7) (end 157.35 101.16) (width 0.25) (layer F.Cu) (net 20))
 (segment (start 155.445 105.605) (end 157.35 103.7) (width 0.25) (layer F.Cu) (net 20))
 (segment (start 140.205 109.415) (end 140.205 97.35) (width 0.25) (layer F.Cu) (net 14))
 (segment (start 144.65 92.905) (end 145.92 92.905) (width 0.25) (layer F.Cu) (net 14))
 (segment (start 140.205 97.35) (end 144.65 92.905) (width 0.25) (layer F.Cu) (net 14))
 (segment (start 148.46 107.51) (end 149.73 108.78) (width 0.25) (layer B.Cu) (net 14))
 (segment (start 140.84 107.51) (end 148.46 107.51) (width 0.25) (layer B.Cu) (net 14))
 (segment (start 140.205 108.145) (end 140.84 107.51) (width 0.25) (layer B.Cu) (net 14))
 (segment (start 140.205 109.415) (end 140.205 108.145) (width 0.25) (layer B.Cu) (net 14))
 (via (at 164.97 85.92) (size 0.8) (drill 0.4) (layers F.Cu B.Cu) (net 10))
 (segment (start 172.59 93.54) (end 164.97 85.92) (width 0.25) (layer F.Cu) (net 10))
 (segment (start 172.59 109.415) (end 172.59 93.54) (width 0.25) (layer F.Cu) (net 10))
 (segment (start 164.97 85.92) (end 164.335 85.285) (width 0.25) (layer B.Cu) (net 10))
 (segment (start 164.335 85.285) (end 152.905 85.285) (width 0.25) (layer B.Cu) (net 10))
 (segment (start 150.365 82.745) (end 145.92 82.745) (width 0.25) (layer B.Cu) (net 10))
 (segment (start 152.905 85.285) (end 150.365 82.745) (width 0.25) (layer B.Cu) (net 10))
 (segment (start 145.92 85.285) (end 130.68 85.285) (width 0.25) (layer B.Cu) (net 11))
 (segment (start 128.14 109.415) (end 128.14 94.175) (width 0.25) (layer F.Cu) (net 11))
 (via (at 128.775 85.92) (size 0.8) (drill 0.4) (layers F.Cu B.Cu) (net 11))
 (segment (start 129.41 85.285) (end 130.68 85.285) (width 0.25) (layer B.Cu) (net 11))
 (segment (start 128.775 85.92) (end 129.41 85.285) (width 0.25) (layer B.Cu) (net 11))
 (segment (start 128.775 85.92) (end 128.775 93.54) (width 0.25) (layer F.Cu) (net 11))
 (segment (start 128.14 94.175) (end 128.775 93.54) (width 0.25) (layer F.Cu) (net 11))
 (segment (start 119.25 88.46) (end 119.25 89.59137) (width 0.25) (layer F.Cu) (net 4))
 (segment (start 123.06 90.365) (end 120.02363 90.365) (width 0.25) (layer F.Cu) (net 4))
 (segment (start 120.02363 90.365) (end 119.954315 90.295685) (width 0.25) (layer F.Cu) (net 4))
 (segment (start 119.25 89.59137) (end 119.954315 90.295685) (width 0.25) (layer F.Cu) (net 4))
 (segment (start 125.6 109.415) (end 125.6 91.635) (width 0.25) (layer F.Cu) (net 4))
 (segment (start 123.06 90.365) (end 124.33 90.365) (width 0.25) (layer F.Cu) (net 4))
 (segment (start 124.33 90.365) (end 125.6 91.635) (width 0.25) (layer F.Cu) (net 4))
 (segment (start 145.92 90.365) (end 128.14 90.365) (width 0.25) (layer B.Cu) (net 13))
 (segment (start 128.14 90.365) (end 124.965 93.54) (width 0.25) (layer B.Cu) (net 13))
 (via (at 124.33 99.89) (size 0.8) (drill 0.4) (layers F.Cu B.Cu) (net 13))
 (segment (start 124.965 99.255) (end 124.33 99.89) (width 0.25) (layer B.Cu) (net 13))
 (segment (start 124.965 93.54) (end 124.965 99.255) (width 0.25) (layer B.Cu) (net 13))
 (segment (start 123.06 101.16) (end 123.06 109.415) (width 0.25) (layer F.Cu) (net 13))
 (segment (start 124.33 99.89) (end 123.06 101.16) (width 0.25) (layer F.Cu) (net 13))
 (segment (start 178.285 76.395) (end 180.21 78.32) (width 0.25) (layer F.Cu) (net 21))
 (segment (start 177.67 76.395) (end 178.285 76.395) (width 0.25) (layer F.Cu) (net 21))
 (segment (start 182.75 84.015) (end 181.48 84.015) (width 0.25) (layer F.Cu) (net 21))
 (segment (start 180.21 82.745) (end 180.21 82.11) (width 0.25) (layer F.Cu) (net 21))
 (segment (start 181.48 84.015) (end 180.21 82.745) (width 0.25) (layer F.Cu) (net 21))
 (segment (start 180.21 78.32) (end 180.21 82.11) (width 0.25) (layer F.Cu) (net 21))
 (segment (start 177.67 74.49) (end 177.87 74.49) (width 0.25) (layer F.Cu) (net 22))
 (segment (start 177.67 73.855) (end 182.75 78.935) (width 0.25) (layer F.Cu) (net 22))
 (segment (start 182.75 78.935) (end 182.75 81.475) (width 0.25) (layer F.Cu) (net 22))
 (segment (start 149.73 101.16) (end 149.73 82.11) (width 0.25) (layer F.Cu) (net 9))
 (segment (start 147.825 80.205) (end 145.92 80.205) (width 0.25) (layer F.Cu) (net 9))
 (segment (start 149.73 82.11) (end 147.825 80.205) (width 0.25) (layer F.Cu) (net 9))
 (segment (start 123.06 93.54) (end 123.26 93.54) (width 0.25) (layer B.Cu) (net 3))
 (segment (start 124.33 92.905) (end 123.06 92.905) (width 0.25) (layer B.Cu) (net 3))
 (segment (start 128.14 89.095) (end 124.33 92.905) (width 0.25) (layer B.Cu) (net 3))
 (segment (start 149.73 89.095) (end 128.14 89.095) (width 0.25) (layer B.Cu) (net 3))
 (segment (start 151 87.825) (end 149.73 89.095) (width 0.25) (layer B.Cu) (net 3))
 (segment (start 177.67 89.095) (end 170.05 89.095) (width 0.25) (layer B.Cu) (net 3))
 (segment (start 168.78 87.825) (end 151 87.825) (width 0.25) (layer B.Cu) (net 3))
 (segment (start 170.05 89.095) (end 168.78 87.825) (width 0.25) (layer B.Cu) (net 3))
 (segment (start 123.675 85.285) (end 124.32 85.93) (width 0.25) (layer F.Cu) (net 6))
 (segment (start 123.06 85.285) (end 123.675 85.285) (width 0.25) (layer F.Cu) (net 6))
 (segment (start 124.31 85.92) (end 124.32 85.93) (width 0.25) (layer F.Cu) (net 6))
 (via (at 127.505 92.27) (size 0.8) (drill 0.4) (layers F.Cu B.Cu) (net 6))
 (segment (start 128.14 91.635) (end 127.505 92.27) (width 0.25) (layer B.Cu) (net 6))
 (segment (start 171.955 91.635) (end 170.685 90.365) (width 0.25) (layer B.Cu) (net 6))
 (segment (start 154.175 91.635) (end 128.14 91.635) (width 0.25) (layer B.Cu) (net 6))
 (segment (start 177.67 91.635) (end 171.955 91.635) (width 0.25) (layer B.Cu) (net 6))
 (segment (start 155.445 90.365) (end 154.175 91.635) (width 0.25) (layer B.Cu) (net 6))
 (segment (start 170.685 90.365) (end 155.445 90.365) (width 0.25) (layer B.Cu) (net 6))
 (segment (start 127.505 89.115) (end 126.86 88.47) (width 0.25) (layer F.Cu) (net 6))
 (segment (start 127.505 92.27) (end 127.505 89.115) (width 0.25) (layer F.Cu) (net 6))
 (segment (start 124.32 85.93) (end 126.86 88.47) (width 0.25) (layer F.Cu) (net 6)))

